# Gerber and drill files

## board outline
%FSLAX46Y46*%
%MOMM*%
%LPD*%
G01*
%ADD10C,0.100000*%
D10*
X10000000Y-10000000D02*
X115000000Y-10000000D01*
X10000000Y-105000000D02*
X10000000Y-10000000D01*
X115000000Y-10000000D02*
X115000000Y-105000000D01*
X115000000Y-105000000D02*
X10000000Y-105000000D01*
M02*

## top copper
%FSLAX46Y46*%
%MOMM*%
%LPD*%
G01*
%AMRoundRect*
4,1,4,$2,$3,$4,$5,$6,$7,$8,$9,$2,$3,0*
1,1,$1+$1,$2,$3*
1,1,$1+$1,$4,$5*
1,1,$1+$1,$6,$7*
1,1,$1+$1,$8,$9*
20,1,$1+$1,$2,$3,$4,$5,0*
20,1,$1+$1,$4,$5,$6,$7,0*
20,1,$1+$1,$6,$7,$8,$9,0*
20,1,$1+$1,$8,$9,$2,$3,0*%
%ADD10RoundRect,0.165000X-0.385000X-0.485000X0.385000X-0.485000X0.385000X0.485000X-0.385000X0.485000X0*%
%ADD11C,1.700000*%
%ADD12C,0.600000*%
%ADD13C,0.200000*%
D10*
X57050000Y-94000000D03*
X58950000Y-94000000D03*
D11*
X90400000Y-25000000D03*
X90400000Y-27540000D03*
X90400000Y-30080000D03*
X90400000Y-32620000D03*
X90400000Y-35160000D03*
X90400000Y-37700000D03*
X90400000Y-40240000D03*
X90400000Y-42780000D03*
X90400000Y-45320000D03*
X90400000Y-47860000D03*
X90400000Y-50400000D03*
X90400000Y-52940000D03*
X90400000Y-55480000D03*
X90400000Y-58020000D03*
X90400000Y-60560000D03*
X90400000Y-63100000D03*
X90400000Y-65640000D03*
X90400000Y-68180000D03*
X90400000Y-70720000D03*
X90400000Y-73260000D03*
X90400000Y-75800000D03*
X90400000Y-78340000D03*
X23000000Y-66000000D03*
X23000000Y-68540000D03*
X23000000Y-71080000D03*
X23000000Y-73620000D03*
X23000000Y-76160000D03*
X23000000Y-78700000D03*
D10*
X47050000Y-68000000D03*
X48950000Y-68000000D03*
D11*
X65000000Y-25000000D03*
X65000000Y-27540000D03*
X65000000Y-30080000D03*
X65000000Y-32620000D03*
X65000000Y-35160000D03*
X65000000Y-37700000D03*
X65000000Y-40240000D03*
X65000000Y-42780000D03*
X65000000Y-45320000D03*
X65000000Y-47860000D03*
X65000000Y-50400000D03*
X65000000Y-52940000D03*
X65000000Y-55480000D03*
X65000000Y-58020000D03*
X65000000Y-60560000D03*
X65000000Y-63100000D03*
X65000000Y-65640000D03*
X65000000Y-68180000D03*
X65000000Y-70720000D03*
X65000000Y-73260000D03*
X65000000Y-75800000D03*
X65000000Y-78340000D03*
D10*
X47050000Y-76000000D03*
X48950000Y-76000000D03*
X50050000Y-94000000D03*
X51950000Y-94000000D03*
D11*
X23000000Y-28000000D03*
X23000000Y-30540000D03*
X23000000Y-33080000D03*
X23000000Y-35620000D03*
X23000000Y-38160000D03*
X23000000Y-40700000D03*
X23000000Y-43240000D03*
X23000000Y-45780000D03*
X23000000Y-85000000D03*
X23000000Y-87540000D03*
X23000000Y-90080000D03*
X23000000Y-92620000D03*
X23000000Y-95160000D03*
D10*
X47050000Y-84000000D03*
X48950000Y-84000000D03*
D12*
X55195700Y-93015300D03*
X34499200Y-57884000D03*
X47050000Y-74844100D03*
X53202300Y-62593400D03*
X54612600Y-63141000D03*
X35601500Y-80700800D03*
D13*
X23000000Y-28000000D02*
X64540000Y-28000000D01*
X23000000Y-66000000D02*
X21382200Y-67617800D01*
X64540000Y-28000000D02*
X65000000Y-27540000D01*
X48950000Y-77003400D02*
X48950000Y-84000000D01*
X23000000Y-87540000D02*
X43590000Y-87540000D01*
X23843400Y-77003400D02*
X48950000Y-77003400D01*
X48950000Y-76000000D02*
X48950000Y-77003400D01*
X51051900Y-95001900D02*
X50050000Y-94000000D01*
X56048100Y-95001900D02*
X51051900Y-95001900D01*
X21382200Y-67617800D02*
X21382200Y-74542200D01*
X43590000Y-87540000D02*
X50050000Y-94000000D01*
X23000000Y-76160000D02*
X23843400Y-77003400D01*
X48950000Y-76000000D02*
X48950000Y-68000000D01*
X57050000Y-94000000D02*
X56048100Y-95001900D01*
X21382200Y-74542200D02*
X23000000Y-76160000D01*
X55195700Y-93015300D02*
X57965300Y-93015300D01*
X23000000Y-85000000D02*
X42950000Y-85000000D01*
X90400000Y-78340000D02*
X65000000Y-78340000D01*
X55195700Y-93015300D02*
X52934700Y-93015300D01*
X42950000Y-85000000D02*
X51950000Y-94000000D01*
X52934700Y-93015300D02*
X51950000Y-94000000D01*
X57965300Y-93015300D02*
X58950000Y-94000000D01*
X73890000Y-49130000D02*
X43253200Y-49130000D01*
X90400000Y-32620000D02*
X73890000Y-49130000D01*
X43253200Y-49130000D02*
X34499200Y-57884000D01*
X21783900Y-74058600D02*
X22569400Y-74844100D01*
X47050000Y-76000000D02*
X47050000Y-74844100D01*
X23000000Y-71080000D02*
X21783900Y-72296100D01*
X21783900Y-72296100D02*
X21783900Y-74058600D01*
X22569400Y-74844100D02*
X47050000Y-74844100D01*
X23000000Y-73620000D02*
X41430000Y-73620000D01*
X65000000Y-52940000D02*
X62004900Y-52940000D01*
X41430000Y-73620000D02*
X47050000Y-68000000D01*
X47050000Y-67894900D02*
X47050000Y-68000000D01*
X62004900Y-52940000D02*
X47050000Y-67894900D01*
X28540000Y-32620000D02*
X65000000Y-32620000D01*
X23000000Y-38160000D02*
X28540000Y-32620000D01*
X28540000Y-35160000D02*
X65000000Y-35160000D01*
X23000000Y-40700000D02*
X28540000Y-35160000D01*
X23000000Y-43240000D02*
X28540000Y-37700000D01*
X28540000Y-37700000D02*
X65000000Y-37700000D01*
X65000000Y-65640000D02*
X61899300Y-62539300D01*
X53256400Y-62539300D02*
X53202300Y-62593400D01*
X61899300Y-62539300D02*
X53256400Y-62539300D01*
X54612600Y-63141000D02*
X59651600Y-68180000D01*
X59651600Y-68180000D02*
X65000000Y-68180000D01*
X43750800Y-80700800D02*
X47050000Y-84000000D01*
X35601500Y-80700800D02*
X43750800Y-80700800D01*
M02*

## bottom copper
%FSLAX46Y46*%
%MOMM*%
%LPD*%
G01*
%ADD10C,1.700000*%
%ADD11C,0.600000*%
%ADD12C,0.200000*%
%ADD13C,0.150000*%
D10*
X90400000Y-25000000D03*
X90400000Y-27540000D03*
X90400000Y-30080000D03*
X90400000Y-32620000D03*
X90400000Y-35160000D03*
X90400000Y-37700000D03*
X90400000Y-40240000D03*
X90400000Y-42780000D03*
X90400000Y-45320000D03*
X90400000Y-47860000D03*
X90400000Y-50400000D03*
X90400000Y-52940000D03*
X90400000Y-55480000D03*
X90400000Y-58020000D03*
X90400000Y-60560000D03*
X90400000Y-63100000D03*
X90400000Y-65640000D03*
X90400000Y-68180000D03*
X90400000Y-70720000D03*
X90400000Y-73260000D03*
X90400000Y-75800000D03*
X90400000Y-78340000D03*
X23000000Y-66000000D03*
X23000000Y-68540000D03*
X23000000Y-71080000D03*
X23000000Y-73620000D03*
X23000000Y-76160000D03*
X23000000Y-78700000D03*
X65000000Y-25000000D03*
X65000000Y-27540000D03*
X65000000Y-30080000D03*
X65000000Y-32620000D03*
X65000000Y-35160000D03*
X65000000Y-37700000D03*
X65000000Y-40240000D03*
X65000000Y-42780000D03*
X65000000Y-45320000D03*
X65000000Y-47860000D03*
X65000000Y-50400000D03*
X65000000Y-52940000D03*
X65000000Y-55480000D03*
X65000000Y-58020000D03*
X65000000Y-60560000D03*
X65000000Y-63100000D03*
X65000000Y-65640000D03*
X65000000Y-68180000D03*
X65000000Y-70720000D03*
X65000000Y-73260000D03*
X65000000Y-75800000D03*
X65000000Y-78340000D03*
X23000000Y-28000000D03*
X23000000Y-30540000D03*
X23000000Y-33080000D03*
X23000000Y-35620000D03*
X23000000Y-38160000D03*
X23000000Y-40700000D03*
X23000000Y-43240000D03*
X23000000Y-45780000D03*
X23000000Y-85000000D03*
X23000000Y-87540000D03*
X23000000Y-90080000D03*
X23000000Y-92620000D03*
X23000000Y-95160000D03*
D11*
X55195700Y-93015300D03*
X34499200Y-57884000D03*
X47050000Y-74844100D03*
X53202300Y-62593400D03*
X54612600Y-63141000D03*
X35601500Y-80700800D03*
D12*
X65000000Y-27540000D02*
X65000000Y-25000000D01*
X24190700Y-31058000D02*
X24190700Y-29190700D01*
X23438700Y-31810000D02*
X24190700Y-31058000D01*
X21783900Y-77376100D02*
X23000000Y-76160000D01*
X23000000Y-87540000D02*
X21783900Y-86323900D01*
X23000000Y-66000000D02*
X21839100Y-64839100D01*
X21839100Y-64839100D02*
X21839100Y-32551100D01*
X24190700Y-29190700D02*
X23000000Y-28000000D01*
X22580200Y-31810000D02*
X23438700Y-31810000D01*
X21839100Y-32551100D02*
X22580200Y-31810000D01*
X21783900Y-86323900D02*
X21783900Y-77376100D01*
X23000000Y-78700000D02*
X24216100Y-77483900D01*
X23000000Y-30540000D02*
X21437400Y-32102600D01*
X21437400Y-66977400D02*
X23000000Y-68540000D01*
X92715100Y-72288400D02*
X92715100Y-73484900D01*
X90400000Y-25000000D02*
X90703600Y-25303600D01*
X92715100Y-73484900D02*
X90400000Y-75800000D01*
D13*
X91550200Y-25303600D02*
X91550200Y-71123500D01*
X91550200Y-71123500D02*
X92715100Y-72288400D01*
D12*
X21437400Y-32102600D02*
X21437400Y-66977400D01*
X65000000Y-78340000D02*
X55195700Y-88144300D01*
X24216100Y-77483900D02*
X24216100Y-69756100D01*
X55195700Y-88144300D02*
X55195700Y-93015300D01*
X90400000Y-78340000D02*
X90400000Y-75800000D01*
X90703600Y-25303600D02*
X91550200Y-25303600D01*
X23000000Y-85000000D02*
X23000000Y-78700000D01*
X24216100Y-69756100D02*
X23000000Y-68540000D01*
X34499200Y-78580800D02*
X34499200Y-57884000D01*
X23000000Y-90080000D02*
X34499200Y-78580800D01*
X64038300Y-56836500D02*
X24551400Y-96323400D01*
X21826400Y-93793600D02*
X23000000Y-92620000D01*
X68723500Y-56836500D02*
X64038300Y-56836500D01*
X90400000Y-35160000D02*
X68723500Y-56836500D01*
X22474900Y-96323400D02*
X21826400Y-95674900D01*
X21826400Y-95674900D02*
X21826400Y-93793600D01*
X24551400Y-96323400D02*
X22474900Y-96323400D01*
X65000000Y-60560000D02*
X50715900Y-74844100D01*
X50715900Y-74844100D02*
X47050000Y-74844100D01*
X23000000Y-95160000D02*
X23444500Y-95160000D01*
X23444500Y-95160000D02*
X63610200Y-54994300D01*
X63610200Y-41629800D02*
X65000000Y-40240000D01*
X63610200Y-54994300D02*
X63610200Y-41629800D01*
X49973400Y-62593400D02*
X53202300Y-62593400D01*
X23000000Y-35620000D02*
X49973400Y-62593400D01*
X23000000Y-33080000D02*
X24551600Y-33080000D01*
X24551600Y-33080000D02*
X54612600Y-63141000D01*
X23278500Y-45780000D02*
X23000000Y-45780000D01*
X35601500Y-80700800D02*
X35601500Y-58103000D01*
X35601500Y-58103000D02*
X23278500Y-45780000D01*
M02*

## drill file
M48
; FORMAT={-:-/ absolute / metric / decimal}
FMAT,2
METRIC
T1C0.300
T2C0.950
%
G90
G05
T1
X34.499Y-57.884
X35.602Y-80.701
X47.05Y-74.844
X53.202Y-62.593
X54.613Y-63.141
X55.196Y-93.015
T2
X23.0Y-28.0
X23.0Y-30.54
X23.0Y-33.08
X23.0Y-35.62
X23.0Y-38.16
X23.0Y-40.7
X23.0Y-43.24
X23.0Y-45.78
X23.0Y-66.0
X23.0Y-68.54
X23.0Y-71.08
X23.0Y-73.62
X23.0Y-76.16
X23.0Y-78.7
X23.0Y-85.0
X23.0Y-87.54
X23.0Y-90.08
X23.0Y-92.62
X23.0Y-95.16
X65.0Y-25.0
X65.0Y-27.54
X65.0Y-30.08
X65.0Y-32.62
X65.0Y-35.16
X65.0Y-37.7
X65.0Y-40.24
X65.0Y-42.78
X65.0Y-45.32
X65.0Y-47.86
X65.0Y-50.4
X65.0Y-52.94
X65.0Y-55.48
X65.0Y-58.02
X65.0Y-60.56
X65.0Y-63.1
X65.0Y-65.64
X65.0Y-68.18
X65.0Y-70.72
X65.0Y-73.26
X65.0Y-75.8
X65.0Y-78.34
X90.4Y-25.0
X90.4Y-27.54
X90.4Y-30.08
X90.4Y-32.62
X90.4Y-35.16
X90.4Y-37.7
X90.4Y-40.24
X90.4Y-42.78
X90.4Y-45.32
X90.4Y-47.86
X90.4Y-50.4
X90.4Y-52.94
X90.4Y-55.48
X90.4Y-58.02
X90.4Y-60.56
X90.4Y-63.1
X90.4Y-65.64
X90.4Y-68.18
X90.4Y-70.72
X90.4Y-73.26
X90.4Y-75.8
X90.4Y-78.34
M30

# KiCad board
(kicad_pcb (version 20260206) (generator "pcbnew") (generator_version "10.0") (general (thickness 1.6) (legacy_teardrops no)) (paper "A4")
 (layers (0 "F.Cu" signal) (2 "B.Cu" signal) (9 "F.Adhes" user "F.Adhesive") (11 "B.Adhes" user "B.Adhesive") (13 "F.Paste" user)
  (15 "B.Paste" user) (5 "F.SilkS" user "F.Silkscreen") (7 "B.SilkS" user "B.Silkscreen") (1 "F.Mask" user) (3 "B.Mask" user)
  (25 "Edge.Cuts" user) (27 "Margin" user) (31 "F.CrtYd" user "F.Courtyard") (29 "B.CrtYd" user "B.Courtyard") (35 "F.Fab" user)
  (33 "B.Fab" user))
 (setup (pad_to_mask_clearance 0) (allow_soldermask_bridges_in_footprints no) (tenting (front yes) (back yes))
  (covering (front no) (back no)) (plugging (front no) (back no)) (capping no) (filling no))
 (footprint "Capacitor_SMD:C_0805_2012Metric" (layer "F.Cu") (at 58 94)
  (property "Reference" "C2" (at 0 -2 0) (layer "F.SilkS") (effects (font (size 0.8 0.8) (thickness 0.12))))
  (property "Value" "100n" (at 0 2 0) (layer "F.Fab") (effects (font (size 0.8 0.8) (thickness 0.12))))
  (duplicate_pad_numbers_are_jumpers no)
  (pad "1" smd roundrect (at -0.95 0) (size 1.1 1.3) (layers "F.Cu" "F.Mask" "F.Paste") (roundrect_rratio 0.15) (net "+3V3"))
  (pad "2" smd roundrect (at 0.95 0) (size 1.1 1.3) (layers "F.Cu" "F.Mask" "F.Paste") (roundrect_rratio 0.15) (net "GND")))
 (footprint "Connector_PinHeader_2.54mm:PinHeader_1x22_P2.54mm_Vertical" (layer "F.Cu") (at 90.4 25)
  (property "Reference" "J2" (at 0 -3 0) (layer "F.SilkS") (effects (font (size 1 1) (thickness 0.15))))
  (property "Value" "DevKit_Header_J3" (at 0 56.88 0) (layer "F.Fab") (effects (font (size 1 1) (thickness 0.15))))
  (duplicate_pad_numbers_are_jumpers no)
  (pad "1" thru_hole circle (at 0 0) (size 1.7 1.7) (drill 0.95) (layers "*.Cu" "*.Mask") (remove_unused_layers no) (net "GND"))
  (pad "2" thru_hole circle (at 0 2.54) (size 1.7 1.7) (drill 0.95) (layers "*.Cu" "*.Mask") (remove_unused_layers no))
  (pad "3" thru_hole circle (at 0 5.08) (size 1.7 1.7) (drill 0.95) (layers "*.Cu" "*.Mask") (remove_unused_layers no))
  (pad "4" thru_hole circle (at 0 7.62) (size 1.7 1.7) (drill 0.95) (layers "*.Cu" "*.Mask") (remove_unused_layers no) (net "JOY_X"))
  (pad "5" thru_hole circle (at 0 10.16) (size 1.7 1.7) (drill 0.95) (layers "*.Cu" "*.Mask") (remove_unused_layers no) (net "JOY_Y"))
  (pad "6" thru_hole circle (at 0 12.7) (size 1.7 1.7) (drill 0.95) (layers "*.Cu" "*.Mask") (remove_unused_layers no))
  (pad "7" thru_hole circle (at 0 15.24) (size 1.7 1.7) (drill 0.95) (layers "*.Cu" "*.Mask") (remove_unused_layers no))
  (pad "8" thru_hole circle (at 0 17.78) (size 1.7 1.7) (drill 0.95) (layers "*.Cu" "*.Mask") (remove_unused_layers no))
  (pad "9" thru_hole circle (at 0 20.32) (size 1.7 1.7) (drill 0.95) (layers "*.Cu" "*.Mask") (remove_unused_layers no))
  (pad "10" thru_hole circle (at 0 22.86) (size 1.7 1.7) (drill 0.95) (layers "*.Cu" "*.Mask") (remove_unused_layers no))
  (pad "11" thru_hole circle (at 0 25.4) (size 1.7 1.7) (drill 0.95) (layers "*.Cu" "*.Mask") (remove_unused_layers no))
  (pad "12" thru_hole circle (at 0 27.94) (size 1.7 1.7) (drill 0.95) (layers "*.Cu" "*.Mask") (remove_unused_layers no))
  (pad "13" thru_hole circle (at 0 30.48) (size 1.7 1.7) (drill 0.95) (layers "*.Cu" "*.Mask") (remove_unused_layers no))
  (pad "14" thru_hole circle (at 0 33.02) (size 1.7 1.7) (drill 0.95) (layers "*.Cu" "*.Mask") (remove_unused_layers no))
  (pad "15" thru_hole circle (at 0 35.56) (size 1.7 1.7) (drill 0.95) (layers "*.Cu" "*.Mask") (remove_unused_layers no))
  (pad "16" thru_hole circle (at 0 38.1) (size 1.7 1.7) (drill 0.95) (layers "*.Cu" "*.Mask") (remove_unused_layers no))
  (pad "17" thru_hole circle (at 0 40.64) (size 1.7 1.7) (drill 0.95) (layers "*.Cu" "*.Mask") (remove_unused_layers no))
  (pad "18" thru_hole circle (at 0 43.18) (size 1.7 1.7) (drill 0.95) (layers "*.Cu" "*.Mask") (remove_unused_layers no))
  (pad "19" thru_hole circle (at 0 45.72) (size 1.7 1.7) (drill 0.95) (layers "*.Cu" "*.Mask") (remove_unused_layers no))
  (pad "20" thru_hole circle (at 0 48.26) (size 1.7 1.7) (drill 0.95) (layers "*.Cu" "*.Mask") (remove_unused_layers no))
  (pad "21" thru_hole circle (at 0 50.8) (size 1.7 1.7) (drill 0.95) (layers "*.Cu" "*.Mask") (remove_unused_layers no) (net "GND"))
  (pad "22" thru_hole circle (at 0 53.34) (size 1.7 1.7) (drill 0.95) (layers "*.Cu" "*.Mask") (remove_unused_layers no) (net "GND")))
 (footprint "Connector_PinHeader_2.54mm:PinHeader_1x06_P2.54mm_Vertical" (layer "F.Cu") (at 23 66)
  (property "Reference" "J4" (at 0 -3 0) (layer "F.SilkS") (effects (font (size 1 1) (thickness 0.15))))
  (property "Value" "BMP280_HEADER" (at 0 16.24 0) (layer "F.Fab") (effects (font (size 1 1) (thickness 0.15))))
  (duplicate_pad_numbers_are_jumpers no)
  (pad "1" thru_hole circle (at 0 0) (size 1.7 1.7) (drill 0.95) (layers "*.Cu" "*.Mask") (remove_unused_layers no) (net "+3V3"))
  (pad "2" thru_hole circle (at 0 2.54) (size 1.7 1.7) (drill 0.95) (layers "*.Cu" "*.Mask") (remove_unused_layers no) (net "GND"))
  (pad "3" thru_hole circle (at 0 5.08) (size 1.7 1.7) (drill 0.95) (layers "*.Cu" "*.Mask") (remove_unused_layers no) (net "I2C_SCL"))
  (pad "4" thru_hole circle (at 0 7.62) (size 1.7 1.7) (drill 0.95) (layers "*.Cu" "*.Mask") (remove_unused_layers no) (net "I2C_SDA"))
  (pad "5" thru_hole circle (at 0 10.16) (size 1.7 1.7) (drill 0.95) (layers "*.Cu" "*.Mask") (remove_unused_layers no) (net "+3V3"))
  (pad "6" thru_hole circle (at 0 12.7) (size 1.7 1.7) (drill 0.95) (layers "*.Cu" "*.Mask") (remove_unused_layers no) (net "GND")))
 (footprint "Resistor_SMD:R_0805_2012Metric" (layer "F.Cu") (at 48 68)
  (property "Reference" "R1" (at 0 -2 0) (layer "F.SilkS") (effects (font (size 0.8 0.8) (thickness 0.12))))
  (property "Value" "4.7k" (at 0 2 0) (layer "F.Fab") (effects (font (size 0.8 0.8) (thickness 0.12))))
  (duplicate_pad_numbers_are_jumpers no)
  (pad "1" smd roundrect (at -0.95 0) (size 1.1 1.3) (layers "F.Cu" "F.Mask" "F.Paste") (roundrect_rratio 0.15) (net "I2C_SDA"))
  (pad "2" smd roundrect (at 0.95 0) (size 1.1 1.3) (layers "F.Cu" "F.Mask" "F.Paste") (roundrect_rratio 0.15) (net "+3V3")))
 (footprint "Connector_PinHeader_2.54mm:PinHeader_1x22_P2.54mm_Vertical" (layer "F.Cu") (at 65 25)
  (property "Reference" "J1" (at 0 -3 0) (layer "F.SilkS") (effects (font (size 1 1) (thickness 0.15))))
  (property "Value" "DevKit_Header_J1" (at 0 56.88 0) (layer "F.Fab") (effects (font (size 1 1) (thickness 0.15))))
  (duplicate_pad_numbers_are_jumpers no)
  (pad "1" thru_hole circle (at 0 0) (size 1.7 1.7) (drill 0.95) (layers "*.Cu" "*.Mask") (remove_unused_layers no) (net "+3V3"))
  (pad "2" thru_hole circle (at 0 2.54) (size 1.7 1.7) (drill 0.95) (layers "*.Cu" "*.Mask") (remove_unused_layers no) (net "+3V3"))
  (pad "3" thru_hole circle (at 0 5.08) (size 1.7 1.7) (drill 0.95) (layers "*.Cu" "*.Mask") (remove_unused_layers no))
  (pad "4" thru_hole circle (at 0 7.62) (size 1.7 1.7) (drill 0.95) (layers "*.Cu" "*.Mask") (remove_unused_layers no) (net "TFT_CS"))
  (pad "5" thru_hole circle (at 0 10.16) (size 1.7 1.7) (drill 0.95) (layers "*.Cu" "*.Mask") (remove_unused_layers no) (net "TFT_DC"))
  (pad "6" thru_hole circle (at 0 12.7) (size 1.7 1.7) (drill 0.95) (layers "*.Cu" "*.Mask") (remove_unused_layers no) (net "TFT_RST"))
  (pad "7" thru_hole circle (at 0 15.24) (size 1.7 1.7) (drill 0.95) (layers "*.Cu" "*.Mask") (remove_unused_layers no) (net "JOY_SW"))
  (pad "8" thru_hole circle (at 0 17.78) (size 1.7 1.7) (drill 0.95) (layers "*.Cu" "*.Mask") (remove_unused_layers no))
  (pad "9" thru_hole circle (at 0 20.32) (size 1.7 1.7) (drill 0.95) (layers "*.Cu" "*.Mask") (remove_unused_layers no))
  (pad "10" thru_hole circle (at 0 22.86) (size 1.7 1.7) (drill 0.95) (layers "*.Cu" "*.Mask") (remove_unused_layers no))
  (pad "11" thru_hole circle (at 0 25.4) (size 1.7 1.7) (drill 0.95) (layers "*.Cu" "*.Mask") (remove_unused_layers no))
  (pad "12" thru_hole circle (at 0 27.94) (size 1.7 1.7) (drill 0.95) (layers "*.Cu" "*.Mask") (remove_unused_layers no) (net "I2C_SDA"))
  (pad "13" thru_hole circle (at 0 30.48) (size 1.7 1.7) (drill 0.95) (layers "*.Cu" "*.Mask") (remove_unused_layers no))
  (pad "14" thru_hole circle (at 0 33.02) (size 1.7 1.7) (drill 0.95) (layers "*.Cu" "*.Mask") (remove_unused_layers no))
  (pad "15" thru_hole circle (at 0 35.56) (size 1.7 1.7) (drill 0.95) (layers "*.Cu" "*.Mask") (remove_unused_layers no) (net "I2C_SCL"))
  (pad "16" thru_hole circle (at 0 38.1) (size 1.7 1.7) (drill 0.95) (layers "*.Cu" "*.Mask") (remove_unused_layers no))
  (pad "17" thru_hole circle (at 0 40.64) (size 1.7 1.7) (drill 0.95) (layers "*.Cu" "*.Mask") (remove_unused_layers no) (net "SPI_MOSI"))
  (pad "18" thru_hole circle (at 0 43.18) (size 1.7 1.7) (drill 0.95) (layers "*.Cu" "*.Mask") (remove_unused_layers no) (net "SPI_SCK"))
  (pad "19" thru_hole circle (at 0 45.72) (size 1.7 1.7) (drill 0.95) (layers "*.Cu" "*.Mask") (remove_unused_layers no))
  (pad "20" thru_hole circle (at 0 48.26) (size 1.7 1.7) (drill 0.95) (layers "*.Cu" "*.Mask") (remove_unused_layers no))
  (pad "21" thru_hole circle (at 0 50.8) (size 1.7 1.7) (drill 0.95) (layers "*.Cu" "*.Mask") (remove_unused_layers no))
  (pad "22" thru_hole circle (at 0 53.34) (size 1.7 1.7) (drill 0.95) (layers "*.Cu" "*.Mask") (remove_unused_layers no) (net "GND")))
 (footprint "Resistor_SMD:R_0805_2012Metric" (layer "F.Cu") (at 48 76)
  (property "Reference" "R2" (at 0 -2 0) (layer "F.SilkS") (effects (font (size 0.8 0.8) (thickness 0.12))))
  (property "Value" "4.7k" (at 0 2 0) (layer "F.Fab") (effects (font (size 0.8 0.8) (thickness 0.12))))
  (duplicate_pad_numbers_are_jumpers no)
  (pad "1" smd roundrect (at -0.95 0) (size 1.1 1.3) (layers "F.Cu" "F.Mask" "F.Paste") (roundrect_rratio 0.15) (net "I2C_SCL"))
  (pad "2" smd roundrect (at 0.95 0) (size 1.1 1.3) (layers "F.Cu" "F.Mask" "F.Paste") (roundrect_rratio 0.15) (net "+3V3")))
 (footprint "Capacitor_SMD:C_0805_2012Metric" (layer "F.Cu") (at 51 94)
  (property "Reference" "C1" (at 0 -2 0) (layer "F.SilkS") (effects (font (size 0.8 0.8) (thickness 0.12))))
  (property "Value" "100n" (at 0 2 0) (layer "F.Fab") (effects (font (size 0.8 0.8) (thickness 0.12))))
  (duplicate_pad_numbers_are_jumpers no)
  (pad "1" smd roundrect (at -0.95 0) (size 1.1 1.3) (layers "F.Cu" "F.Mask" "F.Paste") (roundrect_rratio 0.15) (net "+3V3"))
  (pad "2" smd roundrect (at 0.95 0) (size 1.1 1.3) (layers "F.Cu" "F.Mask" "F.Paste") (roundrect_rratio 0.15) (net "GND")))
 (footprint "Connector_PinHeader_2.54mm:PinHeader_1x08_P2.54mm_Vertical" (layer "F.Cu") (at 23 28)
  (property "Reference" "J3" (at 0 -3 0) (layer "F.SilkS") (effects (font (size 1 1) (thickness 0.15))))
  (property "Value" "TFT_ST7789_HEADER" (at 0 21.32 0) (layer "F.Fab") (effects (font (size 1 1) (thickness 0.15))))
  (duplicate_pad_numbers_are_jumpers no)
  (pad "1" thru_hole circle (at 0 0) (size 1.7 1.7) (drill 0.95) (layers "*.Cu" "*.Mask") (remove_unused_layers no) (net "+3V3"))
  (pad "2" thru_hole circle (at 0 2.54) (size 1.7 1.7) (drill 0.95) (layers "*.Cu" "*.Mask") (remove_unused_layers no) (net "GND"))
  (pad "3" thru_hole circle (at 0 5.08) (size 1.7 1.7) (drill 0.95) (layers "*.Cu" "*.Mask") (remove_unused_layers no) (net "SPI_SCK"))
  (pad "4" thru_hole circle (at 0 7.62) (size 1.7 1.7) (drill 0.95) (layers "*.Cu" "*.Mask") (remove_unused_layers no) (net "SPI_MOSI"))
  (pad "5" thru_hole circle (at 0 10.16) (size 1.7 1.7) (drill 0.95) (layers "*.Cu" "*.Mask") (remove_unused_layers no) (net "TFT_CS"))
  (pad "6" thru_hole circle (at 0 12.7) (size 1.7 1.7) (drill 0.95) (layers "*.Cu" "*.Mask") (remove_unused_layers no) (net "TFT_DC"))
  (pad "7" thru_hole circle (at 0 15.24) (size 1.7 1.7) (drill 0.95) (layers "*.Cu" "*.Mask") (remove_unused_layers no) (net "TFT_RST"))
  (pad "8" thru_hole circle (at 0 17.78) (size 1.7 1.7) (drill 0.95) (layers "*.Cu" "*.Mask") (remove_unused_layers no) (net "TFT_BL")))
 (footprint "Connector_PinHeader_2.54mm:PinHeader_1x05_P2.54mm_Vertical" (layer "F.Cu") (at 23 85)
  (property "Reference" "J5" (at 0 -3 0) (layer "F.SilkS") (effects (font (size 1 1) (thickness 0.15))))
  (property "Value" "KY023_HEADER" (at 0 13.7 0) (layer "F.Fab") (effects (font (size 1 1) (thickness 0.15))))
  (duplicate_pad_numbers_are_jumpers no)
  (pad "1" thru_hole circle (at 0 0) (size 1.7 1.7) (drill 0.95) (layers "*.Cu" "*.Mask") (remove_unused_layers no) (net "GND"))
  (pad "2" thru_hole circle (at 0 2.54) (size 1.7 1.7) (drill 0.95) (layers "*.Cu" "*.Mask") (remove_unused_layers no) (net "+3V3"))
  (pad "3" thru_hole circle (at 0 5.08) (size 1.7 1.7) (drill 0.95) (layers "*.Cu" "*.Mask") (remove_unused_layers no) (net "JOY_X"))
  (pad "4" thru_hole circle (at 0 7.62) (size 1.7 1.7) (drill 0.95) (layers "*.Cu" "*.Mask") (remove_unused_layers no) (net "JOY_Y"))
  (pad "5" thru_hole circle (at 0 10.16) (size 1.7 1.7) (drill 0.95) (layers "*.Cu" "*.Mask") (remove_unused_layers no) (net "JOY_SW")))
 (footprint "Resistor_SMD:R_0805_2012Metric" (layer "F.Cu") (at 48 84)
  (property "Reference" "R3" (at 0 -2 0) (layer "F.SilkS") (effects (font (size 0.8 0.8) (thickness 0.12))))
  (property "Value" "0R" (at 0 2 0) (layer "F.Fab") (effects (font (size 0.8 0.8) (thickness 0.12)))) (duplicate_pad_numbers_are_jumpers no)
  (pad "1" smd roundrect (at -0.95 0) (size 1.1 1.3) (layers "F.Cu" "F.Mask" "F.Paste") (roundrect_rratio 0.15) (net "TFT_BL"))
  (pad "2" smd roundrect (at 0.95 0) (size 1.1 1.3) (layers "F.Cu" "F.Mask" "F.Paste") (roundrect_rratio 0.15) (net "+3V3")))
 (gr_line (start 10 10) (end 115 10) (stroke (width 0.1) (type default)) (layer "Edge.Cuts"))
 (gr_line (start 10 105) (end 10 10) (stroke (width 0.1) (type default)) (layer "Edge.Cuts"))
 (gr_line (start 115 10) (end 115 105) (stroke (width 0.1) (type default)) (layer "Edge.Cuts"))
 (gr_line (start 115 105) (end 10 105) (stroke (width 0.1) (type default)) (layer "Edge.Cuts"))
 (segment (start 23 28) (end 64.54 28) (width 0.2) (layer "F.Cu") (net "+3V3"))
 (segment (start 23 66) (end 21.3822 67.6178) (width 0.2) (layer "F.Cu") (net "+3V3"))
 (segment (start 64.54 28) (end 65 27.54) (width 0.2) (layer "F.Cu") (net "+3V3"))
 (segment (start 48.95 77.0034) (end 48.95 84) (width 0.2) (layer "F.Cu") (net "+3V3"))
 (segment (start 23 87.54) (end 43.59 87.54) (width 0.2) (layer "F.Cu") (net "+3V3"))
 (segment (start 23.8434 77.0034) (end 48.95 77.0034) (width 0.2) (layer "F.Cu") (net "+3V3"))
 (segment (start 48.95 76) (end 48.95 77.0034) (width 0.2) (layer "F.Cu") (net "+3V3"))
 (segment (start 51.0519 95.0019) (end 50.05 94) (width 0.2) (layer "F.Cu") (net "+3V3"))
 (segment (start 56.0481 95.0019) (end 51.0519 95.0019) (width 0.2) (layer "F.Cu") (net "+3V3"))
 (segment (start 21.3822 67.6178) (end 21.3822 74.5422) (width 0.2) (layer "F.Cu") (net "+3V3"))
 (segment (start 43.59 87.54) (end 50.05 94) (width 0.2) (layer "F.Cu") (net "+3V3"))
 (segment (start 23 76.16) (end 23.8434 77.0034) (width 0.2) (layer "F.Cu") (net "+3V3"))
 (segment (start 48.95 76) (end 48.95 68) (width 0.2) (layer "F.Cu") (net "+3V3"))
 (segment (start 57.05 94) (end 56.0481 95.0019) (width 0.2) (layer "F.Cu") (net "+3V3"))
 (segment (start 21.3822 74.5422) (end 23 76.16) (width 0.2) (layer "F.Cu") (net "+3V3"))
 (segment (start 65 27.54) (end 65 25) (width 0.2) (layer "B.Cu") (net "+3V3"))
 (segment (start 24.1907 31.058) (end 24.1907 29.1907) (width 0.2) (layer "B.Cu") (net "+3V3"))
 (segment (start 23.4387 31.81) (end 24.1907 31.058) (width 0.2) (layer "B.Cu") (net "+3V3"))
 (segment (start 21.7839 77.3761) (end 23 76.16) (width 0.2) (layer "B.Cu") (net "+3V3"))
 (segment (start 23 87.54) (end 21.7839 86.3239) (width 0.2) (layer "B.Cu") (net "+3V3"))
 (segment (start 23 66) (end 21.8391 64.8391) (width 0.2) (layer "B.Cu") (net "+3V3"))
 (segment (start 21.8391 64.8391) (end 21.8391 32.5511) (width 0.2) (layer "B.Cu") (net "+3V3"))
 (segment (start 24.1907 29.1907) (end 23 28) (width 0.2) (layer "B.Cu") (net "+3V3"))
 (segment (start 22.5802 31.81) (end 23.4387 31.81) (width 0.2) (layer "B.Cu") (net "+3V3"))
 (segment (start 21.8391 32.5511) (end 22.5802 31.81) (width 0.2) (layer "B.Cu") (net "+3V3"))
 (segment (start 21.7839 86.3239) (end 21.7839 77.3761) (width 0.2) (layer "B.Cu") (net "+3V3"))
 (segment (start 55.1957 93.0153) (end 57.9653 93.0153) (width 0.2) (layer "F.Cu") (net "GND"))
 (segment (start 23 85) (end 42.95 85) (width 0.2) (layer "F.Cu") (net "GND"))
 (segment (start 90.4 78.34) (end 65 78.34) (width 0.2) (layer "F.Cu") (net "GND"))
 (segment (start 55.1957 93.0153) (end 52.9347 93.0153) (width 0.2) (layer "F.Cu") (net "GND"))
 (segment (start 42.95 85) (end 51.95 94) (width 0.2) (layer "F.Cu") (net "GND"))
 (segment (start 52.9347 93.0153) (end 51.95 94) (width 0.2) (layer "F.Cu") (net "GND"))
 (segment (start 57.9653 93.0153) (end 58.95 94) (width 0.2) (layer "F.Cu") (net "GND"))
 (via (at 55.1957 93.0153) (size 0.6) (drill 0.3) (layers "F.Cu" "B.Cu") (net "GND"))
 (segment (start 23 78.7) (end 24.2161 77.4839) (width 0.2) (layer "B.Cu") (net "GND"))
 (segment (start 23 30.54) (end 21.4374 32.1026) (width 0.2) (layer "B.Cu") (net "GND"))
 (segment (start 21.4374 66.9774) (end 23 68.54) (width 0.2) (layer "B.Cu") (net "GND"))
 (segment (start 92.7151 72.2884) (end 92.7151 73.4849) (width 0.2) (layer "B.Cu") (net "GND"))
 (segment (start 90.4 25) (end 90.7036 25.3036) (width 0.2) (layer "B.Cu") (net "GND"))
 (segment (start 92.7151 73.4849) (end 90.4 75.8) (width 0.2) (layer "B.Cu") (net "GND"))
 (segment (start 91.5502 25.3036) (end 91.5502 71.1235) (width 0.15) (layer "B.Cu") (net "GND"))
 (segment (start 91.5502 71.1235) (end 92.7151 72.2884) (width 0.15) (layer "B.Cu") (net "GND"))
 (segment (start 21.4374 32.1026) (end 21.4374 66.9774) (width 0.2) (layer "B.Cu") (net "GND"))
 (segment (start 65 78.34) (end 55.1957 88.1443) (width 0.2) (layer "B.Cu") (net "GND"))
 (segment (start 24.2161 77.4839) (end 24.2161 69.7561) (width 0.2) (layer "B.Cu") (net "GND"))
 (segment (start 55.1957 88.1443) (end 55.1957 93.0153) (width 0.2) (layer "B.Cu") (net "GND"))
 (segment (start 90.4 78.34) (end 90.4 75.8) (width 0.2) (layer "B.Cu") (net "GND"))
 (segment (start 90.7036 25.3036) (end 91.5502 25.3036) (width 0.2) (layer "B.Cu") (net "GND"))
 (segment (start 23 85) (end 23 78.7) (width 0.2) (layer "B.Cu") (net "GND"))
 (segment (start 24.2161 69.7561) (end 23 68.54) (width 0.2) (layer "B.Cu") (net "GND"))
 (segment (start 73.89 49.13) (end 43.2532 49.13) (width 0.2) (layer "F.Cu") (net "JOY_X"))
 (segment (start 90.4 32.62) (end 73.89 49.13) (width 0.2) (layer "F.Cu") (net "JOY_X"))
 (segment (start 43.2532 49.13) (end 34.4992 57.884) (width 0.2) (layer "F.Cu") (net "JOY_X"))
 (via (at 34.4992 57.884) (size 0.6) (drill 0.3) (layers "F.Cu" "B.Cu") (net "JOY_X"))
 (segment (start 34.4992 78.5808) (end 34.4992 57.884) (width 0.2) (layer "B.Cu") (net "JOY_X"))
 (segment (start 23 90.08) (end 34.4992 78.5808) (width 0.2) (layer "B.Cu") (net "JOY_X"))
 (segment (start 64.0383 56.8365) (end 24.5514 96.3234) (width 0.2) (layer "B.Cu") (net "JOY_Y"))
 (segment (start 21.8264 93.7936) (end 23 92.62) (width 0.2) (layer "B.Cu") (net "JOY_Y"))
 (segment (start 68.7235 56.8365) (end 64.0383 56.8365) (width 0.2) (layer "B.Cu") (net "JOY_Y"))
 (segment (start 90.4 35.16) (end 68.7235 56.8365) (width 0.2) (layer "B.Cu") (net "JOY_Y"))
 (segment (start 22.4749 96.3234) (end 21.8264 95.6749) (width 0.2) (layer "B.Cu") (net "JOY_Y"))
 (segment (start 21.8264 95.6749) (end 21.8264 93.7936) (width 0.2) (layer "B.Cu") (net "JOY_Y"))
 (segment (start 24.5514 96.3234) (end 22.4749 96.3234) (width 0.2) (layer "B.Cu") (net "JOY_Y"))
 (segment (start 21.7839 74.0586) (end 22.5694 74.8441) (width 0.2) (layer "F.Cu") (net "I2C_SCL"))
 (segment (start 47.05 76) (end 47.05 74.8441) (width 0.2) (layer "F.Cu") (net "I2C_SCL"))
 (segment (start 23 71.08) (end 21.7839 72.2961) (width 0.2) (layer "F.Cu") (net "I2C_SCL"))
 (segment (start 21.7839 72.2961) (end 21.7839 74.0586) (width 0.2) (layer "F.Cu") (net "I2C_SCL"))
 (segment (start 22.5694 74.8441) (end 47.05 74.8441) (width 0.2) (layer "F.Cu") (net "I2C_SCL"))
 (via (at 47.05 74.8441) (size 0.6) (drill 0.3) (layers "F.Cu" "B.Cu") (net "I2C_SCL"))
 (segment (start 65 60.56) (end 50.7159 74.8441) (width 0.2) (layer "B.Cu") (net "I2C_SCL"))
 (segment (start 50.7159 74.8441) (end 47.05 74.8441) (width 0.2) (layer "B.Cu") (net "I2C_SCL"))
 (segment (start 23 73.62) (end 41.43 73.62) (width 0.2) (layer "F.Cu") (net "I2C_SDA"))
 (segment (start 65 52.94) (end 62.0049 52.94) (width 0.2) (layer "F.Cu") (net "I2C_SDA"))
 (segment (start 41.43 73.62) (end 47.05 68) (width 0.2) (layer "F.Cu") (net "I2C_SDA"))
 (segment (start 47.05 67.8949) (end 47.05 68) (width 0.2) (layer "F.Cu") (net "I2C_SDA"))
 (segment (start 62.0049 52.94) (end 47.05 67.8949) (width 0.2) (layer "F.Cu") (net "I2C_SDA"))
 (segment (start 28.54 32.62) (end 65 32.62) (width 0.2) (layer "F.Cu") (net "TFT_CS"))
 (segment (start 23 38.16) (end 28.54 32.62) (width 0.2) (layer "F.Cu") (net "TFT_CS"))
 (segment (start 28.54 35.16) (end 65 35.16) (width 0.2) (layer "F.Cu") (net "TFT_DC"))
 (segment (start 23 40.7) (end 28.54 35.16) (width 0.2) (layer "F.Cu") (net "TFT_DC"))
 (segment (start 23 43.24) (end 28.54 37.7) (width 0.2) (layer "F.Cu") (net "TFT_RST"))
 (segment (start 28.54 37.7) (end 65 37.7) (width 0.2) (layer "F.Cu") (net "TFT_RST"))
 (segment (start 23 95.16) (end 23.4445 95.16) (width 0.2) (layer "B.Cu") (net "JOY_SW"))
 (segment (start 23.4445 95.16) (end 63.6102 54.9943) (width 0.2) (layer "B.Cu") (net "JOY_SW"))
 (segment (start 63.6102 41.6298) (end 65 40.24) (width 0.2) (layer "B.Cu") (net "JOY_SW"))
 (segment (start 63.6102 54.9943) (end 63.6102 41.6298) (width 0.2) (layer "B.Cu") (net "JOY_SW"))
 (segment (start 65 65.64) (end 61.8993 62.5393) (width 0.2) (layer "F.Cu") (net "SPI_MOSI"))
 (segment (start 53.2564 62.5393) (end 53.2023 62.5934) (width 0.2) (layer "F.Cu") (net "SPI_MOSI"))
 (segment (start 61.8993 62.5393) (end 53.2564 62.5393) (width 0.2) (layer "F.Cu") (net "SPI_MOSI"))
 (via (at 53.2023 62.5934) (size 0.6) (drill 0.3) (layers "F.Cu" "B.Cu") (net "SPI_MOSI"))
 (segment (start 49.9734 62.5934) (end 53.2023 62.5934) (width 0.2) (layer "B.Cu") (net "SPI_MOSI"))
 (segment (start 23 35.62) (end 49.9734 62.5934) (width 0.2) (layer "B.Cu") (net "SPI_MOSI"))
 (segment (start 54.6126 63.141) (end 59.6516 68.18) (width 0.2) (layer "F.Cu") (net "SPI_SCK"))
 (segment (start 59.6516 68.18) (end 65 68.18) (width 0.2) (layer "F.Cu") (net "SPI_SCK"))
 (via (at 54.6126 63.141) (size 0.6) (drill 0.3) (layers "F.Cu" "B.Cu") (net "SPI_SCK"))
 (segment (start 23 33.08) (end 24.5516 33.08) (width 0.2) (layer "B.Cu") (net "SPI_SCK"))
 (segment (start 24.5516 33.08) (end 54.6126 63.141) (width 0.2) (layer "B.Cu") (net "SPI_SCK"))
 (segment (start 43.7508 80.7008) (end 47.05 84) (width 0.2) (layer "F.Cu") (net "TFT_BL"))
 (segment (start 35.6015 80.7008) (end 43.7508 80.7008) (width 0.2) (layer "F.Cu") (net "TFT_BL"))
 (via (at 35.6015 80.7008) (size 0.6) (drill 0.3) (layers "F.Cu" "B.Cu") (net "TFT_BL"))
 (segment (start 23.2785 45.78) (end 23 45.78) (width 0.2) (layer "B.Cu") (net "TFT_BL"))
 (segment (start 35.6015 80.7008) (end 35.6015 58.103) (width 0.2) (layer "B.Cu") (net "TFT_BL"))
 (segment (start 35.6015 58.103) (end 23.2785 45.78) (width 0.2) (layer "B.Cu") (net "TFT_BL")))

